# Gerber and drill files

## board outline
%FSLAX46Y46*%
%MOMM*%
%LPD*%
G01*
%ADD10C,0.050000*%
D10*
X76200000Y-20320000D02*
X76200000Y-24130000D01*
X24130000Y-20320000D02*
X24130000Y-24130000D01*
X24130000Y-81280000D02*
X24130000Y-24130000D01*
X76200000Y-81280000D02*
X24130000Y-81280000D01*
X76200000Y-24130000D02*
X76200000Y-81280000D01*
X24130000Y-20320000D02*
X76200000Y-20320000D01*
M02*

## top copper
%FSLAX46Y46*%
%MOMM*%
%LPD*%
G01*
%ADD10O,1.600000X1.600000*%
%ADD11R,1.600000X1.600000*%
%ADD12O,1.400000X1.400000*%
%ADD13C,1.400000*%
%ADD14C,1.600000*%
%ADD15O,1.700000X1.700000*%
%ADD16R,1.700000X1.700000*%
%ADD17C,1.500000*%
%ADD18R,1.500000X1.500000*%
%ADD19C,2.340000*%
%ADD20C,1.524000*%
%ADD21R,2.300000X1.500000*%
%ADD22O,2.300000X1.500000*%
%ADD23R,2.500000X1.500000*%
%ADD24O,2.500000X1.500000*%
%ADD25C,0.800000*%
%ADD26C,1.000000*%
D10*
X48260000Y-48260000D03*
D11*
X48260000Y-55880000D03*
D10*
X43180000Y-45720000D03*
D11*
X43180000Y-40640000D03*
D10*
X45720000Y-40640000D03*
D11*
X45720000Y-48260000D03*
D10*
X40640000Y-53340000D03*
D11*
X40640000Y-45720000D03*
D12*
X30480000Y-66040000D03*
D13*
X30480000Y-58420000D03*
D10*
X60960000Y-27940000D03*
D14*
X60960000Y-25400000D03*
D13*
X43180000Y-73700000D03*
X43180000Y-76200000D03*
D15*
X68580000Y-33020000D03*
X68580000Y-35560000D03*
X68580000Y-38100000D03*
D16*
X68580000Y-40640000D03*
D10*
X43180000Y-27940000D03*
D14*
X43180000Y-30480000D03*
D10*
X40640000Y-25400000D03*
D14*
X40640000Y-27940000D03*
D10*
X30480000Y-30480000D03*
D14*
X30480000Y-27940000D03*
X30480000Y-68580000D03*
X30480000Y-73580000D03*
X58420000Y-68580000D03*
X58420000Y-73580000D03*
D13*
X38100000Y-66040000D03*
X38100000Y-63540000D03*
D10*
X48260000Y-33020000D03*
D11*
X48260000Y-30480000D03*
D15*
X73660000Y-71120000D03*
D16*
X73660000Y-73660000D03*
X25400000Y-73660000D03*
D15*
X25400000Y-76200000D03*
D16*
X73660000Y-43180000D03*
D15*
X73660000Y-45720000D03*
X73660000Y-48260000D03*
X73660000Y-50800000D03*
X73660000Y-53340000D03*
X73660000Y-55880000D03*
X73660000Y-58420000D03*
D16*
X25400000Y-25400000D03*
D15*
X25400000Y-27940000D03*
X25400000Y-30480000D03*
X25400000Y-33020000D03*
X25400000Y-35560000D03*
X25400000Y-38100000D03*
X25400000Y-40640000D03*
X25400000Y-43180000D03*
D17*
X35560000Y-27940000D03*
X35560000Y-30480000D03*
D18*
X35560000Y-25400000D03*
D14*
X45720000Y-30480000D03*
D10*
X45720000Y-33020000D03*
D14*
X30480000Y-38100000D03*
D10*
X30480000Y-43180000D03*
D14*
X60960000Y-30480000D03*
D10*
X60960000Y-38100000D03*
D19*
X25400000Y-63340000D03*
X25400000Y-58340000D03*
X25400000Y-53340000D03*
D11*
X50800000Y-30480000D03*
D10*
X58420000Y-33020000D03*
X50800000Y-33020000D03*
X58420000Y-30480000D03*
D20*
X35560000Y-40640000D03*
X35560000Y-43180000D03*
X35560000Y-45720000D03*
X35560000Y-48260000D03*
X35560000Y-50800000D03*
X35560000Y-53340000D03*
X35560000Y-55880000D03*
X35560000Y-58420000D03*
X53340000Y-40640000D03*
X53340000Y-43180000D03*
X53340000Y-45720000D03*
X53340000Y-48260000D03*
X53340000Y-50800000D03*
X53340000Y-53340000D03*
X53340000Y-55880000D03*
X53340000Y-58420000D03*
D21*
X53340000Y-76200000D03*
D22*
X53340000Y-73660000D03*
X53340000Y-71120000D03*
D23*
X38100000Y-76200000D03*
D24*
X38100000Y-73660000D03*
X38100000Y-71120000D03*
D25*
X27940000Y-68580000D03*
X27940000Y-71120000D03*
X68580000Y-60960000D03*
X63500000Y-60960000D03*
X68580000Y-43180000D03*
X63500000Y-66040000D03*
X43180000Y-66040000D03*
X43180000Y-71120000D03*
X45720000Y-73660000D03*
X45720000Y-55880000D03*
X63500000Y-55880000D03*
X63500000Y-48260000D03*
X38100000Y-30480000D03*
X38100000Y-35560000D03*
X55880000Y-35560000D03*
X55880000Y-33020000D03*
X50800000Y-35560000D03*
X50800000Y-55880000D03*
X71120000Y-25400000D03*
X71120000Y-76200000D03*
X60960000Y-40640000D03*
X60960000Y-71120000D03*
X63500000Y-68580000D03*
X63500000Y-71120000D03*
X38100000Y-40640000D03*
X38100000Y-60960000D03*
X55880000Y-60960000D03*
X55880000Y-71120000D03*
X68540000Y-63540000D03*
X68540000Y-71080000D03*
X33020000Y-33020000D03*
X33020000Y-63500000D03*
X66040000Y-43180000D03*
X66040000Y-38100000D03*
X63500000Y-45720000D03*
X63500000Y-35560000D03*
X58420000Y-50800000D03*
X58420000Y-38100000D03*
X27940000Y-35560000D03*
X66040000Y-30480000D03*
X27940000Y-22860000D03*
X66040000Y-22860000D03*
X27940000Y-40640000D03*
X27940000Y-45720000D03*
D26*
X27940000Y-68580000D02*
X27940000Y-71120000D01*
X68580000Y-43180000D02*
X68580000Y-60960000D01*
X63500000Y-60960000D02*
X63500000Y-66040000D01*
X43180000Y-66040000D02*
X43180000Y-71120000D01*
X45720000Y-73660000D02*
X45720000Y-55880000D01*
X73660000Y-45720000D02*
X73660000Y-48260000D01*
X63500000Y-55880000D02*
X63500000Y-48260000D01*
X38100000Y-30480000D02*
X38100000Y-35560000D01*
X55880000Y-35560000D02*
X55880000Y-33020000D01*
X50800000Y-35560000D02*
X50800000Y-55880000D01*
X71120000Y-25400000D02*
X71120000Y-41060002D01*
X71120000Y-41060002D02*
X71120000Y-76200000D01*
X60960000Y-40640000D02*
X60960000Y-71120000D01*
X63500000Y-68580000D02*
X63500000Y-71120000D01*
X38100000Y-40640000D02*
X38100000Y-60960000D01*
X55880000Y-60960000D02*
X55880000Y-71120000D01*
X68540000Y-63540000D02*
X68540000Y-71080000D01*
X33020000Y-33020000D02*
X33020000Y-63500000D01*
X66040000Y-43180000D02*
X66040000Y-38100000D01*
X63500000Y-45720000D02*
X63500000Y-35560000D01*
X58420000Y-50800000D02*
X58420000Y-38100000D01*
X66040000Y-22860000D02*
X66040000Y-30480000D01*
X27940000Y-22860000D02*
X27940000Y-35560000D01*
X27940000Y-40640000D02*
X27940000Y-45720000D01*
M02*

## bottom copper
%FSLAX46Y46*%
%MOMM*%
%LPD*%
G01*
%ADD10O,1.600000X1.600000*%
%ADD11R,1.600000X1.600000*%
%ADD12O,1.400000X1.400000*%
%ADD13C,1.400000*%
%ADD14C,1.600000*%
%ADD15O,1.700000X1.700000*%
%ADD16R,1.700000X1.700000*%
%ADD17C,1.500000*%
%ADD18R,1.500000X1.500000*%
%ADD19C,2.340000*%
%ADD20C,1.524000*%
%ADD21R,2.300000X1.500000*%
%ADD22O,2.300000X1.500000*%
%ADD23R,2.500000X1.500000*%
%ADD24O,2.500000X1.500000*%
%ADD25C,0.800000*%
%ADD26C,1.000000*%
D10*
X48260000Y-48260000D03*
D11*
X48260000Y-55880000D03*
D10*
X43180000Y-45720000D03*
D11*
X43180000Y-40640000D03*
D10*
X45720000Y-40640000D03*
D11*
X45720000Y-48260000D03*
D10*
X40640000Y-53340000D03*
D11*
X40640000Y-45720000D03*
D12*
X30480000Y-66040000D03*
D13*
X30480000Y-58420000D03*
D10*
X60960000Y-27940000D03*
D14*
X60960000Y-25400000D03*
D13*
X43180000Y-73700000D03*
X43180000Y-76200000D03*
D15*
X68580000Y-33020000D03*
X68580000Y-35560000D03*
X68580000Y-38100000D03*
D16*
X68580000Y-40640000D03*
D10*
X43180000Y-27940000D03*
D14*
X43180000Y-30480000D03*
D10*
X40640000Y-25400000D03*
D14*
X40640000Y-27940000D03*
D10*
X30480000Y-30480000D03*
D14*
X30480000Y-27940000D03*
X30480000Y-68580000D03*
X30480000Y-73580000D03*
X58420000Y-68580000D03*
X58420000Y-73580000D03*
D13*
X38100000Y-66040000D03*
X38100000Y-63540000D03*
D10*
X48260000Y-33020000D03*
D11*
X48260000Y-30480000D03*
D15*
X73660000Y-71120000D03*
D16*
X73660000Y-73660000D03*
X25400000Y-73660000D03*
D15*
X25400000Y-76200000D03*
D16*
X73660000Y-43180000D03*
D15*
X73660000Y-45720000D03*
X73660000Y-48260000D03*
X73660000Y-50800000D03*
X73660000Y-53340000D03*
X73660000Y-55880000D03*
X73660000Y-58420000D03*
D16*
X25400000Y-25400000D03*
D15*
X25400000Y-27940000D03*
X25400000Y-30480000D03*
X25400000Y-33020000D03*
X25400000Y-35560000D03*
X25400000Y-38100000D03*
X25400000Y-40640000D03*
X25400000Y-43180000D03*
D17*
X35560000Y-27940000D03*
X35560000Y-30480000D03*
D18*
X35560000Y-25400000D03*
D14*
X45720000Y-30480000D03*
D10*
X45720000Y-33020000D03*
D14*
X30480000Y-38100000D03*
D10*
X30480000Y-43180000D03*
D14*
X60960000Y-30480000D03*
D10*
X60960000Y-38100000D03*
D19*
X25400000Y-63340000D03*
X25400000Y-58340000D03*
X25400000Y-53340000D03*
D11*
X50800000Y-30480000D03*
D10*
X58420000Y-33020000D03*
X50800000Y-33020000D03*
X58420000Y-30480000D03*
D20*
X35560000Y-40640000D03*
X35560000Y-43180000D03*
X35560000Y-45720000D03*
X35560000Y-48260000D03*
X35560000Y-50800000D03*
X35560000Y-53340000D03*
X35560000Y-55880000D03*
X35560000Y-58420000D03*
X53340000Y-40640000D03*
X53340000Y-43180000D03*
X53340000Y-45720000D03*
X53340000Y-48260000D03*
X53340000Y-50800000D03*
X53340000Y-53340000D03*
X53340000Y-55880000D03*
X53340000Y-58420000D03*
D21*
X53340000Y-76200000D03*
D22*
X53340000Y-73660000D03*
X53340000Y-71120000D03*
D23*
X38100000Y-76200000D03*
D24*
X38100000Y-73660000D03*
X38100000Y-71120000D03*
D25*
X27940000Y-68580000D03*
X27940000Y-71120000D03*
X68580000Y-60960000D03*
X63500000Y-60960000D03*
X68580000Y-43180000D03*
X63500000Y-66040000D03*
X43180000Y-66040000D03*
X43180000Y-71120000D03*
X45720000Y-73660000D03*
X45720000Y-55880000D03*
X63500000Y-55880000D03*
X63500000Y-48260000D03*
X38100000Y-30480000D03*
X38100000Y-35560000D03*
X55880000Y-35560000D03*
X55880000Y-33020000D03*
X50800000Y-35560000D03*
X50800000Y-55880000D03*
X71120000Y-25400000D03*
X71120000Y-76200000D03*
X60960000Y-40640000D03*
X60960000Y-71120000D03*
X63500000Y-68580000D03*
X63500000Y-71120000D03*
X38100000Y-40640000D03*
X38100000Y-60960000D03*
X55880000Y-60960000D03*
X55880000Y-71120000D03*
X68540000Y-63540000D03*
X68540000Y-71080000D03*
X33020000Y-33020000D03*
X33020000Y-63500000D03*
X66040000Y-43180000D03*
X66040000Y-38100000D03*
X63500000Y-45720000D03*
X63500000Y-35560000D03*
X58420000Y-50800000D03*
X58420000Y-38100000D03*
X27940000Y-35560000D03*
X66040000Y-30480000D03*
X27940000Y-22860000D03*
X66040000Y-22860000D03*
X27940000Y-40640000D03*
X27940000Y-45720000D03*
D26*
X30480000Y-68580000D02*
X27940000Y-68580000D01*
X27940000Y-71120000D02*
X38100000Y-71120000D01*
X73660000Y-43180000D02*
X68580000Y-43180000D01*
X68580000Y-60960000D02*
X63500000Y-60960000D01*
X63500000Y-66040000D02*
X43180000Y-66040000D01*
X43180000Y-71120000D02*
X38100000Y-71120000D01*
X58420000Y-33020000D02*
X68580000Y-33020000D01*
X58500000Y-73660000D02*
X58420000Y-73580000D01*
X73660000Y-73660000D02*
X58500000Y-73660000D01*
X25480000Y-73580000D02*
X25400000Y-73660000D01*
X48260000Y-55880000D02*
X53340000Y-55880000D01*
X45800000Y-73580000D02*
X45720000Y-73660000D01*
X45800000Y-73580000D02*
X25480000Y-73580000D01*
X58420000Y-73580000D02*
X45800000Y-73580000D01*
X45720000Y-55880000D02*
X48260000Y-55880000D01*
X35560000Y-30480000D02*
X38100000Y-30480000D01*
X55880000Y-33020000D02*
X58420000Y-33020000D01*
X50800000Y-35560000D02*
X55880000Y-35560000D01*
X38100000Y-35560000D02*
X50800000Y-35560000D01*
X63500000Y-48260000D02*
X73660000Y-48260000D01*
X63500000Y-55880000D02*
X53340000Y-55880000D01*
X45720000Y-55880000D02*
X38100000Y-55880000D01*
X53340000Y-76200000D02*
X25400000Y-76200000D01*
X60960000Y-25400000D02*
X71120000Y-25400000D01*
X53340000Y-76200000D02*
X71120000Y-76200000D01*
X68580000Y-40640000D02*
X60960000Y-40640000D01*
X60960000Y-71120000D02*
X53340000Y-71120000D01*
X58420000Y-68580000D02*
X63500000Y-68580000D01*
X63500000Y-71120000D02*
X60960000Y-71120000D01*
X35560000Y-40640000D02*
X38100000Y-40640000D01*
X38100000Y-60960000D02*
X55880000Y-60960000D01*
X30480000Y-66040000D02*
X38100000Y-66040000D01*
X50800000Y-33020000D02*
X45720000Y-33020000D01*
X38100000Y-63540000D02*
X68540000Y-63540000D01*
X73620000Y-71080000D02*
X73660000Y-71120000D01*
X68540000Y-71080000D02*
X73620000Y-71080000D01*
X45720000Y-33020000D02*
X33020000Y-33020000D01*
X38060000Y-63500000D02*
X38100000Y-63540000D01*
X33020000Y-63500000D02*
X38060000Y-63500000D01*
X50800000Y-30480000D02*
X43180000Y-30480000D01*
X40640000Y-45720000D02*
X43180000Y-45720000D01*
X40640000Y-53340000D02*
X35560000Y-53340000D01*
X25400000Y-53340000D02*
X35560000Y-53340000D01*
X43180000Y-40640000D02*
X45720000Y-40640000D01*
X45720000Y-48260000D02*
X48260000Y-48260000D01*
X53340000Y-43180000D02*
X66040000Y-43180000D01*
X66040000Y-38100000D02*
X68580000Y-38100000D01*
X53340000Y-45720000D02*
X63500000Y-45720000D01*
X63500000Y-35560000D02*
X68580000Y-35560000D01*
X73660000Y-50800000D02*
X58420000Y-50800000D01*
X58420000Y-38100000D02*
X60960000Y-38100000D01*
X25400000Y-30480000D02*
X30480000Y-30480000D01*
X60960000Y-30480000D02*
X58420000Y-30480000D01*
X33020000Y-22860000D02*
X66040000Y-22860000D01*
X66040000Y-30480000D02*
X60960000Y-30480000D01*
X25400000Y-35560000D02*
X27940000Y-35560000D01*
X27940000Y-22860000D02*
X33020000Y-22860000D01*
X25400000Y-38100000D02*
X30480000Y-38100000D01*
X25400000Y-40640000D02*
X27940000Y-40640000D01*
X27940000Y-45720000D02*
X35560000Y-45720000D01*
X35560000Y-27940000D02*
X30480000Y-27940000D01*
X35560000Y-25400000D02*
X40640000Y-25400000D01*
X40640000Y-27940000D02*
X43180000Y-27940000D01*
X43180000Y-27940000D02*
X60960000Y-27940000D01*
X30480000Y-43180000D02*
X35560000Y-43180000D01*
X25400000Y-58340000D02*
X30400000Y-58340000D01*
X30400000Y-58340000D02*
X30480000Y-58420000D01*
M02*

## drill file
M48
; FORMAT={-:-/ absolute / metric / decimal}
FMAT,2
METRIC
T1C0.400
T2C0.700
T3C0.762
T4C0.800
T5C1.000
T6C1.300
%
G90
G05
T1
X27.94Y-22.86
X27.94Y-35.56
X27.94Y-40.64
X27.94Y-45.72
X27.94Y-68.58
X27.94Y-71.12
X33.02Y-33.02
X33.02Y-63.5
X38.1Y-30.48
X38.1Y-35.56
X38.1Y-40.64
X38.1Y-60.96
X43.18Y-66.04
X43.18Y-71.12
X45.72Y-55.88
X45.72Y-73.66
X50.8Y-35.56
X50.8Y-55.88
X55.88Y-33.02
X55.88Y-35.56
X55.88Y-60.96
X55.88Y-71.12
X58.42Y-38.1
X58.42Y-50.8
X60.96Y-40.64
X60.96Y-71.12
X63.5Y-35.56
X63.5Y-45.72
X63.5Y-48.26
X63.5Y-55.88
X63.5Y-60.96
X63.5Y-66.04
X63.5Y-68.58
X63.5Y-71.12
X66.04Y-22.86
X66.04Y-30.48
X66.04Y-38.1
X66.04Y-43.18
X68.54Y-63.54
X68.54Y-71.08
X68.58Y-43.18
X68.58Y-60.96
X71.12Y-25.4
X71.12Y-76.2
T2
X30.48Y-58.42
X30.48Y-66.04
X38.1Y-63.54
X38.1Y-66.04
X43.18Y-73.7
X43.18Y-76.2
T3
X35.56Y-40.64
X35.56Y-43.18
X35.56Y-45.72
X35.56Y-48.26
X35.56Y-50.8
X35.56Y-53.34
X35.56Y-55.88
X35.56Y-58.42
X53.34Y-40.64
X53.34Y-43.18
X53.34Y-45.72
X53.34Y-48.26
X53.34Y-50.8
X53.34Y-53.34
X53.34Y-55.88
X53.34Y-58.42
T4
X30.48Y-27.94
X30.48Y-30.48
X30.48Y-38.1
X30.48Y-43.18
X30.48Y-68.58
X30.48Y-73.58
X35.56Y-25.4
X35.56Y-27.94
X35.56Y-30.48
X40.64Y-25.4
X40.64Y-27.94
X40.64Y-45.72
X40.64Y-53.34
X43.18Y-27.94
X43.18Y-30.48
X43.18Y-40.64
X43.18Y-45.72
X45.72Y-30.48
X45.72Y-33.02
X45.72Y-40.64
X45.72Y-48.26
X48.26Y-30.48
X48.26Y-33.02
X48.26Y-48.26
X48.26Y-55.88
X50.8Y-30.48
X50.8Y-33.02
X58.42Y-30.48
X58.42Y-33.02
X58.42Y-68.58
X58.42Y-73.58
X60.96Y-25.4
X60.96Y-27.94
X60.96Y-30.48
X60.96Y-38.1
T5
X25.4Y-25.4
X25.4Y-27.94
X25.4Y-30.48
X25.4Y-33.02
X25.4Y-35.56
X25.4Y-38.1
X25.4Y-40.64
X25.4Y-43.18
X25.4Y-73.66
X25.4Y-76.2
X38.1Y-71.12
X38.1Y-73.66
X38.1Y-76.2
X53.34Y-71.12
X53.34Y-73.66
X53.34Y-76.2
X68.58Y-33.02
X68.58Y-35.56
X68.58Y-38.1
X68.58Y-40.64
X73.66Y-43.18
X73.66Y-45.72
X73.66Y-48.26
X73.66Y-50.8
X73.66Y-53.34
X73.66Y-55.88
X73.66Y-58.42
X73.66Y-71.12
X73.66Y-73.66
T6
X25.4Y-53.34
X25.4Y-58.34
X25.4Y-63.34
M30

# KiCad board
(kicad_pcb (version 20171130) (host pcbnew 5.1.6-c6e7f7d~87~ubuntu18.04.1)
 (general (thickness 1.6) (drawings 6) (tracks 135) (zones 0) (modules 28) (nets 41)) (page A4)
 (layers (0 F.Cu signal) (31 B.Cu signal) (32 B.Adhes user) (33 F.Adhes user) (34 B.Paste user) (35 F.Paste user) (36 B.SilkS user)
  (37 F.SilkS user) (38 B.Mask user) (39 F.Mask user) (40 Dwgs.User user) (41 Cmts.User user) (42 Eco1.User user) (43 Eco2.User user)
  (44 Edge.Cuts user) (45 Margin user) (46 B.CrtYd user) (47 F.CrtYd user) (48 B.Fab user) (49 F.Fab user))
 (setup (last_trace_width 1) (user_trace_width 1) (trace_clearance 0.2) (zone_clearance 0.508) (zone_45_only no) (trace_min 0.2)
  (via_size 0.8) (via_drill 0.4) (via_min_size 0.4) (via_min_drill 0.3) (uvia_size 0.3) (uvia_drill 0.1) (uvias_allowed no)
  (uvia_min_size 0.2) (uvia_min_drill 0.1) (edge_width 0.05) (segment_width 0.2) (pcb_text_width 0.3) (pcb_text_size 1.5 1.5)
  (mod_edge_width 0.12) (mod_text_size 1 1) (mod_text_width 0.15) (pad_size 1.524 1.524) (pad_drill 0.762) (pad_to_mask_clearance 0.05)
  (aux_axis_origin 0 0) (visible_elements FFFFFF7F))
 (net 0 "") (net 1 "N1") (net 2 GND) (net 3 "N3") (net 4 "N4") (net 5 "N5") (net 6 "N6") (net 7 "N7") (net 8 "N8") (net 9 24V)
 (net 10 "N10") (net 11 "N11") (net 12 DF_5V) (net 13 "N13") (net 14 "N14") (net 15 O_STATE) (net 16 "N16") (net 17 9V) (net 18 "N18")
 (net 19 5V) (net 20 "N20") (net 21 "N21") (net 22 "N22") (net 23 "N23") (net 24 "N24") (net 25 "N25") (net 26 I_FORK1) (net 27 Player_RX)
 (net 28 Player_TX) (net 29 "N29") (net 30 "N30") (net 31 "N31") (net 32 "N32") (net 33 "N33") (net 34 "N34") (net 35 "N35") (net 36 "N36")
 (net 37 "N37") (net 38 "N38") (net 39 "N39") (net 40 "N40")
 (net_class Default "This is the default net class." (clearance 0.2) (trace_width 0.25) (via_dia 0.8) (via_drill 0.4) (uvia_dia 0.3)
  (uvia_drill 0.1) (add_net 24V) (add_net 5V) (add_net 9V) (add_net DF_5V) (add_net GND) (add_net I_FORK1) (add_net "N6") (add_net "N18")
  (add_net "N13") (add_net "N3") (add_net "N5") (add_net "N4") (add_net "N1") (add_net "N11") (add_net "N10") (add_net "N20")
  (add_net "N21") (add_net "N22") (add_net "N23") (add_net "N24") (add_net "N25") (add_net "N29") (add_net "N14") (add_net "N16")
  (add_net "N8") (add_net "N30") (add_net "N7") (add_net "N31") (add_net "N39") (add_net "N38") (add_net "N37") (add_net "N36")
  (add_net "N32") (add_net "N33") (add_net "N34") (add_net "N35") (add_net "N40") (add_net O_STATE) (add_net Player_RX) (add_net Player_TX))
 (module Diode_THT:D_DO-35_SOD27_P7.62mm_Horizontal (layer F.Cu) (at 48.26 55.88 90)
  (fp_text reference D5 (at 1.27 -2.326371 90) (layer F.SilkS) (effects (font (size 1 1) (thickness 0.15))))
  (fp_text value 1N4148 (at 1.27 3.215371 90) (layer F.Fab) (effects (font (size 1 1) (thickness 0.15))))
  (pad 2 thru_hole oval (at 7.62 0 90) (size 1.6 1.6) (drill 0.8) (layers *.Cu *.Mask) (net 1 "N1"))
  (pad 1 thru_hole rect (at 0 0 90) (size 1.6 1.6) (drill 0.8) (layers *.Cu *.Mask) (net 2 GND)))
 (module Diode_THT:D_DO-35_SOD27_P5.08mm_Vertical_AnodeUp (layer F.Cu) (at 43.18 40.64 270)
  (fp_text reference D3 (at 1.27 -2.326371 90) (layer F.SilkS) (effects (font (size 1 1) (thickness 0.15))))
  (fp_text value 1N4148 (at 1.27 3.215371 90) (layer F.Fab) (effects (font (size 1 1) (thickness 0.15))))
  (pad 2 thru_hole oval (at 5.08 0 270) (size 1.6 1.6) (drill 0.8) (layers *.Cu *.Mask) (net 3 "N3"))
  (pad 1 thru_hole rect (at 0 0 270) (size 1.6 1.6) (drill 0.8) (layers *.Cu *.Mask) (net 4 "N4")))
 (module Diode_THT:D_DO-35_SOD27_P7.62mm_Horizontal (layer F.Cu) (at 45.72 48.26 90)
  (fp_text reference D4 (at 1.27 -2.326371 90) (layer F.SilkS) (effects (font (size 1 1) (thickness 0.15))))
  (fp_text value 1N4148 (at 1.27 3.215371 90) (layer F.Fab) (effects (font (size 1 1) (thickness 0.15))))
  (pad 2 thru_hole oval (at 7.62 0 90) (size 1.6 1.6) (drill 0.8) (layers *.Cu *.Mask) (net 4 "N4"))
  (pad 1 thru_hole rect (at 0 0 90) (size 1.6 1.6) (drill 0.8) (layers *.Cu *.Mask) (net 1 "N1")))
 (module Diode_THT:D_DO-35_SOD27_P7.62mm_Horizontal (layer F.Cu) (at 40.64 45.72 270)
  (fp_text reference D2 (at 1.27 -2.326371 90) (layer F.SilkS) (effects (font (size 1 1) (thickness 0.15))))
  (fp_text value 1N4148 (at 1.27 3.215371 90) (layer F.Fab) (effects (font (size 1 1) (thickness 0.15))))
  (pad 2 thru_hole oval (at 7.62 0 270) (size 1.6 1.6) (drill 0.8) (layers *.Cu *.Mask) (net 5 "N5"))
  (pad 1 thru_hole rect (at 0 0 270) (size 1.6 1.6) (drill 0.8) (layers *.Cu *.Mask) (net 3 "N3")))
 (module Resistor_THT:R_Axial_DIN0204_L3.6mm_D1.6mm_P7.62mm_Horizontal (layer F.Cu) (at 30.48 58.42 270)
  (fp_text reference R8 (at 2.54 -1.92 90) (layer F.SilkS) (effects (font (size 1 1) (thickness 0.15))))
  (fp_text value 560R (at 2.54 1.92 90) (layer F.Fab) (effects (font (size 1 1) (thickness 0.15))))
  (pad 2 thru_hole oval (at 7.62 0 270) (size 1.4 1.4) (drill 0.7) (layers *.Cu *.Mask) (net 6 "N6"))
  (pad 1 thru_hole circle (at 0 0 270) (size 1.4 1.4) (drill 0.7) (layers *.Cu *.Mask) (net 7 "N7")))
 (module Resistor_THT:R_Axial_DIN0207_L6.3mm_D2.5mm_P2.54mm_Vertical (layer F.Cu) (at 60.96 25.4 270)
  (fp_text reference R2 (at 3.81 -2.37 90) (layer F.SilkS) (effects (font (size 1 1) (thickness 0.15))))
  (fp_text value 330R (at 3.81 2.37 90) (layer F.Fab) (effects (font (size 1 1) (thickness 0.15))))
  (pad 2 thru_hole oval (at 2.54 0 270) (size 1.6 1.6) (drill 0.8) (layers *.Cu *.Mask) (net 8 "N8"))
  (pad 1 thru_hole circle (at 0 0 270) (size 1.6 1.6) (drill 0.8) (layers *.Cu *.Mask) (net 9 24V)))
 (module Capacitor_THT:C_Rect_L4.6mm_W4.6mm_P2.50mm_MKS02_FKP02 (layer F.Cu) (at 43.18 76.2 90)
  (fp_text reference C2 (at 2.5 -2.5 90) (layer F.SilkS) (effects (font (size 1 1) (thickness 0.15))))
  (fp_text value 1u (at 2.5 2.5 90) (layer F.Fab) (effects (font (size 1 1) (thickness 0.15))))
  (pad 2 thru_hole circle (at 2.5 0 90) (size 1.4 1.4) (drill 0.7) (layers *.Cu *.Mask) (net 2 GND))
  (pad 1 thru_hole circle (at 0 0 90) (size 1.4 1.4) (drill 0.7) (layers *.Cu *.Mask) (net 9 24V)))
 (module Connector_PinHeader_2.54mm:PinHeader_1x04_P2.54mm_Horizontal (layer B.Cu) (at 68.58 40.64)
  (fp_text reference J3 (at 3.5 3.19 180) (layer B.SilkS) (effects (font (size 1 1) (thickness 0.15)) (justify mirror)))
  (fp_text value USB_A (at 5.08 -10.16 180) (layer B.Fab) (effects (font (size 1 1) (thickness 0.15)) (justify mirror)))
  (pad 4 thru_hole oval (at 0 -7.62) (size 1.7 1.7) (drill 1) (layers *.Cu *.Mask) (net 2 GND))
  (pad 3 thru_hole oval (at 0 -5.08) (size 1.7 1.7) (drill 1) (layers *.Cu *.Mask) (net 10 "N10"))
  (pad 2 thru_hole oval (at 0 -2.54) (size 1.7 1.7) (drill 1) (layers *.Cu *.Mask) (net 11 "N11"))
  (pad 1 thru_hole rect (at 0 0) (size 1.7 1.7) (drill 1) (layers *.Cu *.Mask) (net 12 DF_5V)))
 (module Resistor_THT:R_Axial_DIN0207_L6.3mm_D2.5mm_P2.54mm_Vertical (layer F.Cu) (at 43.18 30.48 90)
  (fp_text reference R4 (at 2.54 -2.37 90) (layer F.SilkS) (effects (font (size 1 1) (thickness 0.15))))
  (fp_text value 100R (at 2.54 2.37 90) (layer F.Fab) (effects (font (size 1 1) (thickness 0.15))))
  (pad 2 thru_hole oval (at 2.54 0 90) (size 1.6 1.6) (drill 0.8) (layers *.Cu *.Mask) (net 8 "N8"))
  (pad 1 thru_hole circle (at 0 0 90) (size 1.6 1.6) (drill 0.8) (layers *.Cu *.Mask) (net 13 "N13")))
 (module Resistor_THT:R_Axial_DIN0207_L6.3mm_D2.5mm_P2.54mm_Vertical (layer F.Cu) (at 40.64 27.94 90)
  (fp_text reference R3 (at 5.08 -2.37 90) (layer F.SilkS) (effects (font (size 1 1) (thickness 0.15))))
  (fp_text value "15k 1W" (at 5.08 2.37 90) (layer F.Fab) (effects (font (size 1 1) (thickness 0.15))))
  (pad 2 thru_hole oval (at 2.54 0 90) (size 1.6 1.6) (drill 0.8) (layers *.Cu *.Mask) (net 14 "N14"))
  (pad 1 thru_hole circle (at 0 0 90) (size 1.6 1.6) (drill 0.8) (layers *.Cu *.Mask) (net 8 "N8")))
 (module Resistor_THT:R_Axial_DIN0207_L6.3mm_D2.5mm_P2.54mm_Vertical (layer F.Cu) (at 30.48 27.94 270)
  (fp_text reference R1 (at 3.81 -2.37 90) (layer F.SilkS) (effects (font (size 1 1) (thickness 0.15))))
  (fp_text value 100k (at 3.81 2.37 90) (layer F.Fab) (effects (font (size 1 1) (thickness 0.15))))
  (pad 2 thru_hole oval (at 2.54 0 270) (size 1.6 1.6) (drill 0.8) (layers *.Cu *.Mask) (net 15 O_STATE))
  (pad 1 thru_hole circle (at 0 0 270) (size 1.6 1.6) (drill 0.8) (layers *.Cu *.Mask) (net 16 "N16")))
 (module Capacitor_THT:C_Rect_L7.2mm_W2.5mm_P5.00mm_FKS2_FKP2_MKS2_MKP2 (layer F.Cu) (at 30.48 68.58 270)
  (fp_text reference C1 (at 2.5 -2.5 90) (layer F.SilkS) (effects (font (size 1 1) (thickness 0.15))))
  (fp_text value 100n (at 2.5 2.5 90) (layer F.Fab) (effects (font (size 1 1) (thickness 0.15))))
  (pad 1 thru_hole circle (at 0 0 270) (size 1.6 1.6) (drill 0.8) (layers *.Cu *.Mask) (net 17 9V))
  (pad 2 thru_hole circle (at 5 0 270) (size 1.6 1.6) (drill 0.8) (layers *.Cu *.Mask) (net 2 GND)))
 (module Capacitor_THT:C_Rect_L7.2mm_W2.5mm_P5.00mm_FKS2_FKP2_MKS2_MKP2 (layer F.Cu) (at 58.42 68.58 270)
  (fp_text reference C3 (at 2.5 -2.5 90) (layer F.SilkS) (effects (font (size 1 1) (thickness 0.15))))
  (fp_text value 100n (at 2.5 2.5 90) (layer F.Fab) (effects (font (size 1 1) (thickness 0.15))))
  (pad 1 thru_hole circle (at 0 0 270) (size 1.6 1.6) (drill 0.8) (layers *.Cu *.Mask) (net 12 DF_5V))
  (pad 2 thru_hole circle (at 5 0 270) (size 1.6 1.6) (drill 0.8) (layers *.Cu *.Mask) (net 2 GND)))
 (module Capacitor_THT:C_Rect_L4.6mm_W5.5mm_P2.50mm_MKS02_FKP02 (layer F.Cu) (at 38.1 66.04 90)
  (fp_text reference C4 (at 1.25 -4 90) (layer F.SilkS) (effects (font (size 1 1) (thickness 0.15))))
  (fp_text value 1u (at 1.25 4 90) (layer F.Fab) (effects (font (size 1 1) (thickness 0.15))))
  (pad 1 thru_hole circle (at 0 0 90) (size 1.4 1.4) (drill 0.7) (layers *.Cu *.Mask) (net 6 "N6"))
  (pad 2 thru_hole circle (at 2.5 0 90) (size 1.4 1.4) (drill 0.7) (layers *.Cu *.Mask) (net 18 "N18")))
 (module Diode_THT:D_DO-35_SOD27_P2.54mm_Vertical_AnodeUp (layer F.Cu) (at 48.26 30.48 270)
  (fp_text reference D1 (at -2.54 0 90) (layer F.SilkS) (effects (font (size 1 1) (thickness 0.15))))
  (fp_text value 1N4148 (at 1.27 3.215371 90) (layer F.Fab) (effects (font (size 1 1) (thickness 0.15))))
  (pad 2 thru_hole oval (at 2.54 0 270) (size 1.6 1.6) (drill 0.8) (layers *.Cu *.Mask) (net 18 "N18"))
  (pad 1 thru_hole rect (at 0 0 270) (size 1.6 1.6) (drill 0.8) (layers *.Cu *.Mask) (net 13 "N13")))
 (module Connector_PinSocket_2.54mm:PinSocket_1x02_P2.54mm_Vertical (layer F.Cu) (at 73.66 73.66 180)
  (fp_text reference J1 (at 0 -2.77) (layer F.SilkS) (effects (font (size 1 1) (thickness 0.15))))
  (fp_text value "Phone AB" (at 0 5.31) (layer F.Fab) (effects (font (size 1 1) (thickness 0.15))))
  (pad 2 thru_hole oval (at 0 2.54 180) (size 1.7 1.7) (drill 1) (layers *.Cu *.Mask) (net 18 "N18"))
  (pad 1 thru_hole rect (at 0 0 180) (size 1.7 1.7) (drill 1) (layers *.Cu *.Mask) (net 2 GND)))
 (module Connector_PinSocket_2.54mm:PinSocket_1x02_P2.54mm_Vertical (layer F.Cu) (at 25.4 73.66)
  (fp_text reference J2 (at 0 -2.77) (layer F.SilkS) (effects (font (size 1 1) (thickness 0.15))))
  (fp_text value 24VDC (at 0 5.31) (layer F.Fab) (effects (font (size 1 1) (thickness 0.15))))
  (pad 1 thru_hole rect (at 0 0) (size 1.7 1.7) (drill 1) (layers *.Cu *.Mask) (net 2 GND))
  (pad 2 thru_hole oval (at 0 2.54) (size 1.7 1.7) (drill 1) (layers *.Cu *.Mask) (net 9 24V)))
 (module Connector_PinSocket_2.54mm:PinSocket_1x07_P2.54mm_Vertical (layer F.Cu) (at 73.66 43.18)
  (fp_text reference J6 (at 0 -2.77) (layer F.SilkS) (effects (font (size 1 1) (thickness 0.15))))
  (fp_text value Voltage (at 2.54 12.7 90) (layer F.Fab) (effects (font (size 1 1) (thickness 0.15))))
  (pad 1 thru_hole rect (at 0 0) (size 1.7 1.7) (drill 1) (layers *.Cu *.Mask) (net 17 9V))
  (pad 2 thru_hole oval (at 0 2.54) (size 1.7 1.7) (drill 1) (layers *.Cu *.Mask) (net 2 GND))
  (pad 3 thru_hole oval (at 0 5.08) (size 1.7 1.7) (drill 1) (layers *.Cu *.Mask) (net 2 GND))
  (pad 4 thru_hole oval (at 0 7.62) (size 1.7 1.7) (drill 1) (layers *.Cu *.Mask) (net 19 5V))
  (pad 5 thru_hole oval (at 0 10.16) (size 1.7 1.7) (drill 1) (layers *.Cu *.Mask) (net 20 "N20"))
  (pad 6 thru_hole oval (at 0 12.7) (size 1.7 1.7) (drill 1) (layers *.Cu *.Mask) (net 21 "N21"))
  (pad 7 thru_hole oval (at 0 15.24) (size 1.7 1.7) (drill 1) (layers *.Cu *.Mask) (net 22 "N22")))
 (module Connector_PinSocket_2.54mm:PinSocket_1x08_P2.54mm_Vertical (layer F.Cu) (at 25.4 25.4)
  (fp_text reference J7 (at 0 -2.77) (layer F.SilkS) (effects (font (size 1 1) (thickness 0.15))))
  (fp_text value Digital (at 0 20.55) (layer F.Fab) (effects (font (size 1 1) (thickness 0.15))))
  (pad 1 thru_hole rect (at 0 0) (size 1.7 1.7) (drill 1) (layers *.Cu *.Mask) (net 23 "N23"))
  (pad 2 thru_hole oval (at 0 2.54) (size 1.7 1.7) (drill 1) (layers *.Cu *.Mask) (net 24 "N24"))
  (pad 3 thru_hole oval (at 0 5.08) (size 1.7 1.7) (drill 1) (layers *.Cu *.Mask) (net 15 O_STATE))
  (pad 4 thru_hole oval (at 0 7.62) (size 1.7 1.7) (drill 1) (layers *.Cu *.Mask) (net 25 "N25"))
  (pad 5 thru_hole oval (at 0 10.16) (size 1.7 1.7) (drill 1) (layers *.Cu *.Mask) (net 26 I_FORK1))
  (pad 6 thru_hole oval (at 0 12.7) (size 1.7 1.7) (drill 1) (layers *.Cu *.Mask) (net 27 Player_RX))
  (pad 7 thru_hole oval (at 0 15.24) (size 1.7 1.7) (drill 1) (layers *.Cu *.Mask) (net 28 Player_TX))
  (pad 8 thru_hole oval (at 0 17.78) (size 1.7 1.7) (drill 1) (layers *.Cu *.Mask) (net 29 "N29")))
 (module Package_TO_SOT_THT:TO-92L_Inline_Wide (layer F.Cu) (at 35.56 25.4 270)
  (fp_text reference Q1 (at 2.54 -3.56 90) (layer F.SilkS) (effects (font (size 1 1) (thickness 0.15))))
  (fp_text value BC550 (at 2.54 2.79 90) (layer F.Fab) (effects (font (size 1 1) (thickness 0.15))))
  (pad 2 thru_hole circle (at 2.54 0) (size 1.5 1.5) (drill 0.8) (layers *.Cu *.Mask) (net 16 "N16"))
  (pad 3 thru_hole circle (at 5.08 0) (size 1.5 1.5) (drill 0.8) (layers *.Cu *.Mask) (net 2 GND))
  (pad 1 thru_hole rect (at 0 0) (size 1.5 1.5) (drill 0.8) (layers *.Cu *.Mask) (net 14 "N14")))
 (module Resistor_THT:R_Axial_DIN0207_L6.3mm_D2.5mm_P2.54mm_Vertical (layer F.Cu) (at 45.72 30.48 270)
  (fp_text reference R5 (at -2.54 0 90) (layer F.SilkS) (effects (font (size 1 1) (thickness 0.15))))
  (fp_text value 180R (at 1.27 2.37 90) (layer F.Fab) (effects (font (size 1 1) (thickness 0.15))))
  (pad 1 thru_hole circle (at 0 0 270) (size 1.6 1.6) (drill 0.8) (layers *.Cu *.Mask) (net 13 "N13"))
  (pad 2 thru_hole oval (at 2.54 0 270) (size 1.6 1.6) (drill 0.8) (layers *.Cu *.Mask) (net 18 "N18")))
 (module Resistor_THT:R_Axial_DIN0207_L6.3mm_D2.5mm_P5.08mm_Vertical (layer F.Cu) (at 30.48 38.1 270)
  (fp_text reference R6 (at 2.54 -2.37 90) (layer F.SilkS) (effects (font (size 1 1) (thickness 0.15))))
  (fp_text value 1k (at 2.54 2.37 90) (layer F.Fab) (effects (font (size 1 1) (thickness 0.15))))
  (pad 1 thru_hole circle (at 0 0 270) (size 1.6 1.6) (drill 0.8) (layers *.Cu *.Mask) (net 27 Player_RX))
  (pad 2 thru_hole oval (at 5.08 0 270) (size 1.6 1.6) (drill 0.8) (layers *.Cu *.Mask) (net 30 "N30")))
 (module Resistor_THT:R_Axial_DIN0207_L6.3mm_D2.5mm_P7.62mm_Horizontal (layer F.Cu) (at 60.96 30.48 270)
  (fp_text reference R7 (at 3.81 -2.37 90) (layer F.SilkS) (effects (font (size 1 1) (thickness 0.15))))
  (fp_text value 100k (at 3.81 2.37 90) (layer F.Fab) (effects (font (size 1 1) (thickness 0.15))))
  (pad 1 thru_hole circle (at 0 0 270) (size 1.6 1.6) (drill 0.8) (layers *.Cu *.Mask) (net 26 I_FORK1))
  (pad 2 thru_hole oval (at 7.62 0 270) (size 1.6 1.6) (drill 0.8) (layers *.Cu *.Mask) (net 19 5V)))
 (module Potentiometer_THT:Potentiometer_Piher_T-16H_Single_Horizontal (layer F.Cu) (at 25.4 53.34 180)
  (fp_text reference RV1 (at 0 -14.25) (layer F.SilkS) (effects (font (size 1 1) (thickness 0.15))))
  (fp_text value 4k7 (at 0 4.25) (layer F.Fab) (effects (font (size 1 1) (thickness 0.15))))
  (pad 3 thru_hole circle (at 0 -10 180) (size 2.34 2.34) (drill 1.3) (layers *.Cu *.Mask) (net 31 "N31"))
  (pad 2 thru_hole circle (at 0 -5 180) (size 2.34 2.34) (drill 1.3) (layers *.Cu *.Mask) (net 7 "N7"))
  (pad 1 thru_hole circle (at 0 0 180) (size 2.34 2.34) (drill 1.3) (layers *.Cu *.Mask) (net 5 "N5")))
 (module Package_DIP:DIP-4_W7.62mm (layer F.Cu) (at 50.8 30.48)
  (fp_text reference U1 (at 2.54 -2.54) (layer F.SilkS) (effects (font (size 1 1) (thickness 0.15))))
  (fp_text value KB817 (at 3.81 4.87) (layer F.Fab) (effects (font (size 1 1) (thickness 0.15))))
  (pad 1 thru_hole rect (at 0 0) (size 1.6 1.6) (drill 0.8) (layers *.Cu *.Mask) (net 13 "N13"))
  (pad 3 thru_hole oval (at 7.62 2.54) (size 1.6 1.6) (drill 0.8) (layers *.Cu *.Mask) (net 2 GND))
  (pad 2 thru_hole oval (at 0 2.54) (size 1.6 1.6) (drill 0.8) (layers *.Cu *.Mask) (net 18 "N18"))
  (pad 4 thru_hole oval (at 7.62 0) (size 1.6 1.6) (drill 0.8) (layers *.Cu *.Mask) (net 26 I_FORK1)))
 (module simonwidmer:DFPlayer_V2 (layer F.Cu) (at 43.18 40.64)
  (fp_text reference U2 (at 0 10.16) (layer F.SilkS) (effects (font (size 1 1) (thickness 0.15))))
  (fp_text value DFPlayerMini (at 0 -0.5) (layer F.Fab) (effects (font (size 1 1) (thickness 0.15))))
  (pad 1 thru_hole circle (at -7.62 0) (size 1.524 1.524) (drill 0.762) (layers *.Cu *.Mask) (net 12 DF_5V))
  (pad 2 thru_hole circle (at -7.62 2.54) (size 1.524 1.524) (drill 0.762) (layers *.Cu *.Mask) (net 30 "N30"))
  (pad 3 thru_hole circle (at -7.62 5.08) (size 1.524 1.524) (drill 0.762) (layers *.Cu *.Mask) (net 28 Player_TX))
  (pad 4 thru_hole circle (at -7.62 7.62) (size 1.524 1.524) (drill 0.762) (layers *.Cu *.Mask) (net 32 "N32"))
  (pad 5 thru_hole circle (at -7.62 10.16) (size 1.524 1.524) (drill 0.762) (layers *.Cu *.Mask) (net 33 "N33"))
  (pad 6 thru_hole circle (at -7.62 12.7) (size 1.524 1.524) (drill 0.762) (layers *.Cu *.Mask) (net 5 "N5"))
  (pad 7 thru_hole circle (at -7.62 15.24) (size 1.524 1.524) (drill 0.762) (layers *.Cu *.Mask) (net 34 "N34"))
  (pad 8 thru_hole circle (at -7.62 17.78) (size 1.524 1.524) (drill 0.762) (layers *.Cu *.Mask) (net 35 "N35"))
  (pad 16 thru_hole circle (at 10.16 0) (size 1.524 1.524) (drill 0.762) (layers *.Cu *.Mask) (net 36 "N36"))
  (pad 15 thru_hole circle (at 10.16 2.54) (size 1.524 1.524) (drill 0.762) (layers *.Cu *.Mask) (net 11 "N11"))
  (pad 14 thru_hole circle (at 10.16 5.08) (size 1.524 1.524) (drill 0.762) (layers *.Cu *.Mask) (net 10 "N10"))
  (pad 13 thru_hole circle (at 10.16 7.62) (size 1.524 1.524) (drill 0.762) (layers *.Cu *.Mask) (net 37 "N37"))
  (pad 12 thru_hole circle (at 10.16 10.16) (size 1.524 1.524) (drill 0.762) (layers *.Cu *.Mask) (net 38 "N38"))
  (pad 11 thru_hole circle (at 10.16 12.7) (size 1.524 1.524) (drill 0.762) (layers *.Cu *.Mask) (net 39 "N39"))
  (pad 10 thru_hole circle (at 10.16 15.24) (size 1.524 1.524) (drill 0.762) (layers *.Cu *.Mask) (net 2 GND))
  (pad 9 thru_hole circle (at 10.16 17.78) (size 1.524 1.524) (drill 0.762) (layers *.Cu *.Mask) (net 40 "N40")))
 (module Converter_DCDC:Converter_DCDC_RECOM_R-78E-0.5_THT (layer F.Cu) (at 53.34 76.2 90)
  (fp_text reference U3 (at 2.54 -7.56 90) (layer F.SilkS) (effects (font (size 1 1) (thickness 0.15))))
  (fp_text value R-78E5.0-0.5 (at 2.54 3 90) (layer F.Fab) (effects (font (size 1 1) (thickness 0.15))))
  (pad 1 thru_hole rect (at 0 0 90) (size 1.5 2.3) (drill 1) (layers *.Cu *.Mask) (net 9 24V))
  (pad 2 thru_hole oval (at 2.54 0 90) (size 1.5 2.3) (drill 1) (layers *.Cu *.Mask) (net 2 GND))
  (pad 3 thru_hole oval (at 5.08 0 90) (size 1.5 2.3) (drill 1) (layers *.Cu *.Mask) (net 12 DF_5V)))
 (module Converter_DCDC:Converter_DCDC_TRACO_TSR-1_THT (layer F.Cu) (at 38.1 76.2 90)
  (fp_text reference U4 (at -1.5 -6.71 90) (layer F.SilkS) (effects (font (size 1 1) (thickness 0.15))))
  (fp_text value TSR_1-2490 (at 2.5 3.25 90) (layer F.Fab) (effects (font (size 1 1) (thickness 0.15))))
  (pad 1 thru_hole rect (at 0 0 90) (size 1.5 2.5) (drill 1) (layers *.Cu *.Mask) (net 9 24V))
  (pad 2 thru_hole oval (at 2.54 0 90) (size 1.5 2.5) (drill 1) (layers *.Cu *.Mask) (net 2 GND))
  (pad 3 thru_hole oval (at 5.08 0 90) (size 1.5 2.5) (drill 1) (layers *.Cu *.Mask) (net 17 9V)))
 (gr_line (start 76.2 20.32) (end 76.2 24.13) (layer Edge.Cuts) (width 0.05))
 (gr_line (start 24.13 20.32) (end 24.13 24.13) (layer Edge.Cuts) (width 0.05))
 (gr_line (start 24.13 81.28) (end 24.13 24.13) (layer Edge.Cuts) (width 0.05))
 (gr_line (start 76.2 81.28) (end 24.13 81.28) (layer Edge.Cuts) (width 0.05))
 (gr_line (start 76.2 24.13) (end 76.2 81.28) (layer Edge.Cuts) (width 0.05))
 (gr_line (start 24.13 20.32) (end 76.2 20.32) (layer Edge.Cuts) (width 0.05))
 (segment (start 30.48 68.58) (end 27.94 68.58) (width 1) (layer B.Cu) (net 17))
 (via (at 27.94 68.58) (size 0.8) (drill 0.4) (layers F.Cu B.Cu) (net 17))
 (segment (start 27.94 68.58) (end 27.94 71.12) (width 1) (layer F.Cu) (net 17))
 (via (at 27.94 71.12) (size 0.8) (drill 0.4) (layers F.Cu B.Cu) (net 17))
 (segment (start 27.94 71.12) (end 38.1 71.12) (width 1) (layer B.Cu) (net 17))
 (via (at 68.58 60.96) (size 0.8) (drill 0.4) (layers F.Cu B.Cu) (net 17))
 (segment (start 68.58 43.18) (end 68.58 60.96) (width 1) (layer F.Cu) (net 17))
 (via (at 63.5 60.96) (size 0.8) (drill 0.4) (layers F.Cu B.Cu) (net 17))
 (segment (start 73.66 43.18) (end 68.58 43.18) (width 1) (layer B.Cu) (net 17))
 (segment (start 68.58 60.96) (end 63.5 60.96) (width 1) (layer B.Cu) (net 17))
 (via (at 68.58 43.18) (size 0.8) (drill 0.4) (layers F.Cu B.Cu) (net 17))
 (segment (start 63.5 60.96) (end 63.5 66.04) (width 1) (layer F.Cu) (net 17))
 (via (at 63.5 66.04) (size 0.8) (drill 0.4) (layers F.Cu B.Cu) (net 17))
 (segment (start 63.5 66.04) (end 43.18 66.04) (width 1) (layer B.Cu) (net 17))
 (via (at 43.18 66.04) (size 0.8) (drill 0.4) (layers F.Cu B.Cu) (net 17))
 (segment (start 43.18 66.04) (end 43.18 71.12) (width 1) (layer F.Cu) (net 17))
 (via (at 43.18 71.12) (size 0.8) (drill 0.4) (layers F.Cu B.Cu) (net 17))
 (segment (start 43.18 71.12) (end 38.1 71.12) (width 1) (layer B.Cu) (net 17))
 (segment (start 58.42 33.02) (end 68.58 33.02) (width 1) (layer B.Cu) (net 2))
 (segment (start 58.5 73.66) (end 58.42 73.58) (width 1) (layer B.Cu) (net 2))
 (segment (start 73.66 73.66) (end 58.5 73.66) (width 1) (layer B.Cu) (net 2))
 (segment (start 25.48 73.58) (end 25.4 73.66) (width 1) (layer B.Cu) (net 2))
 (segment (start 48.26 55.88) (end 53.34 55.88) (width 1) (layer B.Cu) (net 2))
 (via (at 45.72 73.66) (size 0.8) (drill 0.4) (layers F.Cu B.Cu) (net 2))
 (segment (start 45.8 73.58) (end 45.72 73.66) (width 1) (layer B.Cu) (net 2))
 (segment (start 45.8 73.58) (end 25.48 73.58) (width 1) (layer B.Cu) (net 2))
 (segment (start 58.42 73.58) (end 45.8 73.58) (width 1) (layer B.Cu) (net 2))
 (segment (start 45.72 73.66) (end 45.72 55.88) (width 1) (layer F.Cu) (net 2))
 (via (at 45.72 55.88) (size 0.8) (drill 0.4) (layers F.Cu B.Cu) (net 2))
 (segment (start 45.72 55.88) (end 48.26 55.88) (width 1) (layer B.Cu) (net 2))
 (segment (start 73.66 45.72) (end 73.66 48.26) (width 1) (layer F.Cu) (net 2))
 (via (at 63.5 55.88) (size 0.8) (drill 0.4) (layers F.Cu B.Cu) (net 2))
 (segment (start 63.5 55.88) (end 63.5 48.26) (width 1) (layer F.Cu) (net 2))
 (via (at 63.5 48.26) (size 0.8) (drill 0.4) (layers F.Cu B.Cu) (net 2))
 (segment (start 35.56 30.48) (end 38.1 30.48) (width 1) (layer B.Cu) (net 2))
 (via (at 38.1 30.48) (size 0.8) (drill 0.4) (layers F.Cu B.Cu) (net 2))
 (segment (start 38.1 30.48) (end 38.1 35.56) (width 1) (layer F.Cu) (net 2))
 (via (at 38.1 35.56) (size 0.8) (drill 0.4) (layers F.Cu B.Cu) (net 2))
 (via (at 55.88 35.56) (size 0.8) (drill 0.4) (layers F.Cu B.Cu) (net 2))
 (segment (start 55.88 35.56) (end 55.88 33.02) (width 1) (layer F.Cu) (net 2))
 (via (at 55.88 33.02) (size 0.8) (drill 0.4) (layers F.Cu B.Cu) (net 2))
 (segment (start 55.88 33.02) (end 58.42 33.02) (width 1) (layer B.Cu) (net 2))
 (via (at 50.8 35.56) (size 0.8) (drill 0.4) (layers F.Cu B.Cu) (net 2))
 (segment (start 50.8 35.56) (end 55.88 35.56) (width 1) (layer B.Cu) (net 2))
 (segment (start 38.1 35.56) (end 50.8 35.56) (width 1) (layer B.Cu) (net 2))
 (segment (start 50.8 35.56) (end 50.8 55.88) (width 1) (layer F.Cu) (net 2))
 (via (at 50.8 55.88) (size 0.8) (drill 0.4) (layers F.Cu B.Cu) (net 2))
 (segment (start 63.5 48.26) (end 73.66 48.26) (width 1) (layer B.Cu) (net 2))
 (segment (start 63.5 55.88) (end 53.34 55.88) (width 1) (layer B.Cu) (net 2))
 (segment (start 45.72 55.88) (end 38.1 55.88) (width 1) (layer B.Cu) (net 2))
 (segment (start 53.34 76.2) (end 25.4 76.2) (width 1) (layer B.Cu) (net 9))
 (segment (start 60.96 25.4) (end 71.12 25.4) (width 1) (layer B.Cu) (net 9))
 (via (at 71.12 25.4) (size 0.8) (drill 0.4) (layers F.Cu B.Cu) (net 9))
 (segment (start 71.12 25.4) (end 71.12 41.060002) (width 1) (layer F.Cu) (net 9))
 (via (at 71.12 76.2) (size 0.8) (drill 0.4) (layers F.Cu B.Cu) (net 9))
 (segment (start 71.12 41.060002) (end 71.12 76.2) (width 1) (layer F.Cu) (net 9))
 (segment (start 53.34 76.2) (end 71.12 76.2) (width 1) (layer B.Cu) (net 9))
 (segment (start 68.58 40.64) (end 60.96 40.64) (width 1) (layer B.Cu) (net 12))
 (via (at 60.96 40.64) (size 0.8) (drill 0.4) (layers F.Cu B.Cu) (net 12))
 (segment (start 60.96 40.64) (end 60.96 71.12) (width 1) (layer F.Cu) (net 12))
 (via (at 60.96 71.12) (size 0.8) (drill 0.4) (layers F.Cu B.Cu) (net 12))
 (segment (start 60.96 71.12) (end 53.34 71.12) (width 1) (layer B.Cu) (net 12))
 (segment (start 58.42 68.58) (end 63.5 68.58) (width 1) (layer B.Cu) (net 12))
 (via (at 63.5 68.58) (size 0.8) (drill 0.4) (layers F.Cu B.Cu) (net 12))
 (segment (start 63.5 68.58) (end 63.5 71.12) (width 1) (layer F.Cu) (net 12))
 (via (at 63.5 71.12) (size 0.8) (drill 0.4) (layers F.Cu B.Cu) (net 12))
 (segment (start 63.5 71.12) (end 60.96 71.12) (width 1) (layer B.Cu) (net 12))
 (segment (start 35.56 40.64) (end 38.1 40.64) (width 1) (layer B.Cu) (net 12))
 (via (at 38.1 40.64) (size 0.8) (drill 0.4) (layers F.Cu B.Cu) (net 12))
 (segment (start 38.1 40.64) (end 38.1 60.96) (width 1) (layer F.Cu) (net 12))
 (via (at 38.1 60.96) (size 0.8) (drill 0.4) (layers F.Cu B.Cu) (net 12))
 (segment (start 38.1 60.96) (end 55.88 60.96) (width 1) (layer B.Cu) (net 12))
 (via (at 55.88 60.96) (size 0.8) (drill 0.4) (layers F.Cu B.Cu) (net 12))
 (segment (start 55.88 60.96) (end 55.88 71.12) (width 1) (layer F.Cu) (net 12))
 (via (at 55.88 71.12) (size 0.8) (drill 0.4) (layers F.Cu B.Cu) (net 12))
 (segment (start 30.48 66.04) (end 38.1 66.04) (width 1) (layer B.Cu) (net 6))
 (segment (start 50.8 33.02) (end 45.72 33.02) (width 1) (layer B.Cu) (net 18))
 (segment (start 38.1 63.54) (end 68.54 63.54) (width 1) (layer B.Cu) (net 18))
 (via (at 68.54 63.54) (size 0.8) (drill 0.4) (layers F.Cu B.Cu) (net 18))
 (segment (start 68.54 63.54) (end 68.54 71.08) (width 1) (layer F.Cu) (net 18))
 (via (at 68.54 71.08) (size 0.8) (drill 0.4) (layers F.Cu B.Cu) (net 18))
 (segment (start 73.62 71.08) (end 73.66 71.12) (width 1) (layer B.Cu) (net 18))
 (segment (start 68.54 71.08) (end 73.62 71.08) (width 1) (layer B.Cu) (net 18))
 (segment (start 45.72 33.02) (end 33.02 33.02) (width 1) (layer B.Cu) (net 18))
 (via (at 33.02 33.02) (size 0.8) (drill 0.4) (layers F.Cu B.Cu) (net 18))
 (segment (start 33.02 33.02) (end 33.02 63.5) (width 1) (layer F.Cu) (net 18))
 (via (at 33.02 63.5) (size 0.8) (drill 0.4) (layers F.Cu B.Cu) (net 18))
 (segment (start 38.06 63.5) (end 38.1 63.54) (width 1) (layer B.Cu) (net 18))
 (segment (start 33.02 63.5) (end 38.06 63.5) (width 1) (layer B.Cu) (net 18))
 (segment (start 50.8 30.48) (end 43.18 30.48) (width 1) (layer B.Cu) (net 13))
 (segment (start 40.64 45.72) (end 43.18 45.72) (width 1) (layer B.Cu) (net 3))
 (segment (start 40.64 53.34) (end 35.56 53.34) (width 1) (layer B.Cu) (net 5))
 (segment (start 25.4 53.34) (end 35.56 53.34) (width 1) (layer B.Cu) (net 5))
 (segment (start 43.18 40.64) (end 45.72 40.64) (width 1) (layer B.Cu) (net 4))
 (segment (start 45.72 48.26) (end 48.26 48.26) (width 1) (layer B.Cu) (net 1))
 (segment (start 53.34 43.18) (end 66.04 43.18) (width 1) (layer B.Cu) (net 11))
 (via (at 66.04 43.18) (size 0.8) (drill 0.4) (layers F.Cu B.Cu) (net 11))
 (segment (start 66.04 43.18) (end 66.04 38.1) (width 1) (layer F.Cu) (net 11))
 (via (at 66.04 38.1) (size 0.8) (drill 0.4) (layers F.Cu B.Cu) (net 11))
 (segment (start 66.04 38.1) (end 68.58 38.1) (width 1) (layer B.Cu) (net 11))
 (segment (start 53.34 45.72) (end 63.5 45.72) (width 1) (layer B.Cu) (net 10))
 (via (at 63.5 45.72) (size 0.8) (drill 0.4) (layers F.Cu B.Cu) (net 10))
 (segment (start 63.5 45.72) (end 63.5 35.56) (width 1) (layer F.Cu) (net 10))
 (via (at 63.5 35.56) (size 0.8) (drill 0.4) (layers F.Cu B.Cu) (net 10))
 (segment (start 63.5 35.56) (end 68.58 35.56) (width 1) (layer B.Cu) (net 10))
 (segment (start 73.66 50.8) (end 58.42 50.8) (width 1) (layer B.Cu) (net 19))
 (via (at 58.42 50.8) (size 0.8) (drill 0.4) (layers F.Cu B.Cu) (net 19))
 (segment (start 58.42 50.8) (end 58.42 38.1) (width 1) (layer F.Cu) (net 19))
 (via (at 58.42 38.1) (size 0.8) (drill 0.4) (layers F.Cu B.Cu) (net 19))
 (segment (start 58.42 38.1) (end 60.96 38.1) (width 1) (layer B.Cu) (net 19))
 (segment (start 25.4 30.48) (end 30.48 30.48) (width 1) (layer B.Cu) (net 15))
 (segment (start 60.96 30.48) (end 58.42 30.48) (width 1) (layer B.Cu) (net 26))
 (segment (start 33.02 22.86) (end 66.04 22.86) (width 1) (layer B.Cu) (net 26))
 (via (at 27.94 35.56) (size 0.8) (drill 0.4) (layers F.Cu B.Cu) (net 26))
 (via (at 66.04 30.48) (size 0.8) (drill 0.4) (layers F.Cu B.Cu) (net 26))
 (segment (start 66.04 30.48) (end 60.96 30.48) (width 1) (layer B.Cu) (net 26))
 (via (at 27.94 22.86) (size 0.8) (drill 0.4) (layers F.Cu B.Cu) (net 26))
 (segment (start 66.04 22.86) (end 66.04 30.48) (width 1) (layer F.Cu) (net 26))
 (via (at 66.04 22.86) (size 0.8) (drill 0.4) (layers F.Cu B.Cu) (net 26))
 (segment (start 25.4 35.56) (end 27.94 35.56) (width 1) (layer B.Cu) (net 26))
 (segment (start 27.94 22.86) (end 33.02 22.86) (width 1) (layer B.Cu) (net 26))
 (segment (start 27.94 22.86) (end 27.94 35.56) (width 1) (layer F.Cu) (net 26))
 (segment (start 25.4 38.1) (end 30.48 38.1) (width 1) (layer B.Cu) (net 27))
 (segment (start 25.4 40.64) (end 27.94 40.64) (width 1) (layer B.Cu) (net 28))
 (via (at 27.94 40.64) (size 0.8) (drill 0.4) (layers F.Cu B.Cu) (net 28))
 (segment (start 27.94 40.64) (end 27.94 45.72) (width 1) (layer F.Cu) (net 28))
 (via (at 27.94 45.72) (size 0.8) (drill 0.4) (layers F.Cu B.Cu) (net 28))
 (segment (start 27.94 45.72) (end 35.56 45.72) (width 1) (layer B.Cu) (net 28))
 (segment (start 35.56 27.94) (end 30.48 27.94) (width 1) (layer B.Cu) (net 16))
 (segment (start 35.56 25.4) (end 40.64 25.4) (width 1) (layer B.Cu) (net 14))
 (segment (start 40.64 27.94) (end 43.18 27.94) (width 1) (layer B.Cu) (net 8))
 (segment (start 43.18 27.94) (end 60.96 27.94) (width 1) (layer B.Cu) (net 8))
 (segment (start 30.48 43.18) (end 35.56 43.18) (width 1) (layer B.Cu) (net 30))
 (segment (start 25.4 58.34) (end 30.4 58.34) (width 1) (layer B.Cu) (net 7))
 (segment (start 30.4 58.34) (end 30.48 58.42) (width 1) (layer B.Cu) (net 7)))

